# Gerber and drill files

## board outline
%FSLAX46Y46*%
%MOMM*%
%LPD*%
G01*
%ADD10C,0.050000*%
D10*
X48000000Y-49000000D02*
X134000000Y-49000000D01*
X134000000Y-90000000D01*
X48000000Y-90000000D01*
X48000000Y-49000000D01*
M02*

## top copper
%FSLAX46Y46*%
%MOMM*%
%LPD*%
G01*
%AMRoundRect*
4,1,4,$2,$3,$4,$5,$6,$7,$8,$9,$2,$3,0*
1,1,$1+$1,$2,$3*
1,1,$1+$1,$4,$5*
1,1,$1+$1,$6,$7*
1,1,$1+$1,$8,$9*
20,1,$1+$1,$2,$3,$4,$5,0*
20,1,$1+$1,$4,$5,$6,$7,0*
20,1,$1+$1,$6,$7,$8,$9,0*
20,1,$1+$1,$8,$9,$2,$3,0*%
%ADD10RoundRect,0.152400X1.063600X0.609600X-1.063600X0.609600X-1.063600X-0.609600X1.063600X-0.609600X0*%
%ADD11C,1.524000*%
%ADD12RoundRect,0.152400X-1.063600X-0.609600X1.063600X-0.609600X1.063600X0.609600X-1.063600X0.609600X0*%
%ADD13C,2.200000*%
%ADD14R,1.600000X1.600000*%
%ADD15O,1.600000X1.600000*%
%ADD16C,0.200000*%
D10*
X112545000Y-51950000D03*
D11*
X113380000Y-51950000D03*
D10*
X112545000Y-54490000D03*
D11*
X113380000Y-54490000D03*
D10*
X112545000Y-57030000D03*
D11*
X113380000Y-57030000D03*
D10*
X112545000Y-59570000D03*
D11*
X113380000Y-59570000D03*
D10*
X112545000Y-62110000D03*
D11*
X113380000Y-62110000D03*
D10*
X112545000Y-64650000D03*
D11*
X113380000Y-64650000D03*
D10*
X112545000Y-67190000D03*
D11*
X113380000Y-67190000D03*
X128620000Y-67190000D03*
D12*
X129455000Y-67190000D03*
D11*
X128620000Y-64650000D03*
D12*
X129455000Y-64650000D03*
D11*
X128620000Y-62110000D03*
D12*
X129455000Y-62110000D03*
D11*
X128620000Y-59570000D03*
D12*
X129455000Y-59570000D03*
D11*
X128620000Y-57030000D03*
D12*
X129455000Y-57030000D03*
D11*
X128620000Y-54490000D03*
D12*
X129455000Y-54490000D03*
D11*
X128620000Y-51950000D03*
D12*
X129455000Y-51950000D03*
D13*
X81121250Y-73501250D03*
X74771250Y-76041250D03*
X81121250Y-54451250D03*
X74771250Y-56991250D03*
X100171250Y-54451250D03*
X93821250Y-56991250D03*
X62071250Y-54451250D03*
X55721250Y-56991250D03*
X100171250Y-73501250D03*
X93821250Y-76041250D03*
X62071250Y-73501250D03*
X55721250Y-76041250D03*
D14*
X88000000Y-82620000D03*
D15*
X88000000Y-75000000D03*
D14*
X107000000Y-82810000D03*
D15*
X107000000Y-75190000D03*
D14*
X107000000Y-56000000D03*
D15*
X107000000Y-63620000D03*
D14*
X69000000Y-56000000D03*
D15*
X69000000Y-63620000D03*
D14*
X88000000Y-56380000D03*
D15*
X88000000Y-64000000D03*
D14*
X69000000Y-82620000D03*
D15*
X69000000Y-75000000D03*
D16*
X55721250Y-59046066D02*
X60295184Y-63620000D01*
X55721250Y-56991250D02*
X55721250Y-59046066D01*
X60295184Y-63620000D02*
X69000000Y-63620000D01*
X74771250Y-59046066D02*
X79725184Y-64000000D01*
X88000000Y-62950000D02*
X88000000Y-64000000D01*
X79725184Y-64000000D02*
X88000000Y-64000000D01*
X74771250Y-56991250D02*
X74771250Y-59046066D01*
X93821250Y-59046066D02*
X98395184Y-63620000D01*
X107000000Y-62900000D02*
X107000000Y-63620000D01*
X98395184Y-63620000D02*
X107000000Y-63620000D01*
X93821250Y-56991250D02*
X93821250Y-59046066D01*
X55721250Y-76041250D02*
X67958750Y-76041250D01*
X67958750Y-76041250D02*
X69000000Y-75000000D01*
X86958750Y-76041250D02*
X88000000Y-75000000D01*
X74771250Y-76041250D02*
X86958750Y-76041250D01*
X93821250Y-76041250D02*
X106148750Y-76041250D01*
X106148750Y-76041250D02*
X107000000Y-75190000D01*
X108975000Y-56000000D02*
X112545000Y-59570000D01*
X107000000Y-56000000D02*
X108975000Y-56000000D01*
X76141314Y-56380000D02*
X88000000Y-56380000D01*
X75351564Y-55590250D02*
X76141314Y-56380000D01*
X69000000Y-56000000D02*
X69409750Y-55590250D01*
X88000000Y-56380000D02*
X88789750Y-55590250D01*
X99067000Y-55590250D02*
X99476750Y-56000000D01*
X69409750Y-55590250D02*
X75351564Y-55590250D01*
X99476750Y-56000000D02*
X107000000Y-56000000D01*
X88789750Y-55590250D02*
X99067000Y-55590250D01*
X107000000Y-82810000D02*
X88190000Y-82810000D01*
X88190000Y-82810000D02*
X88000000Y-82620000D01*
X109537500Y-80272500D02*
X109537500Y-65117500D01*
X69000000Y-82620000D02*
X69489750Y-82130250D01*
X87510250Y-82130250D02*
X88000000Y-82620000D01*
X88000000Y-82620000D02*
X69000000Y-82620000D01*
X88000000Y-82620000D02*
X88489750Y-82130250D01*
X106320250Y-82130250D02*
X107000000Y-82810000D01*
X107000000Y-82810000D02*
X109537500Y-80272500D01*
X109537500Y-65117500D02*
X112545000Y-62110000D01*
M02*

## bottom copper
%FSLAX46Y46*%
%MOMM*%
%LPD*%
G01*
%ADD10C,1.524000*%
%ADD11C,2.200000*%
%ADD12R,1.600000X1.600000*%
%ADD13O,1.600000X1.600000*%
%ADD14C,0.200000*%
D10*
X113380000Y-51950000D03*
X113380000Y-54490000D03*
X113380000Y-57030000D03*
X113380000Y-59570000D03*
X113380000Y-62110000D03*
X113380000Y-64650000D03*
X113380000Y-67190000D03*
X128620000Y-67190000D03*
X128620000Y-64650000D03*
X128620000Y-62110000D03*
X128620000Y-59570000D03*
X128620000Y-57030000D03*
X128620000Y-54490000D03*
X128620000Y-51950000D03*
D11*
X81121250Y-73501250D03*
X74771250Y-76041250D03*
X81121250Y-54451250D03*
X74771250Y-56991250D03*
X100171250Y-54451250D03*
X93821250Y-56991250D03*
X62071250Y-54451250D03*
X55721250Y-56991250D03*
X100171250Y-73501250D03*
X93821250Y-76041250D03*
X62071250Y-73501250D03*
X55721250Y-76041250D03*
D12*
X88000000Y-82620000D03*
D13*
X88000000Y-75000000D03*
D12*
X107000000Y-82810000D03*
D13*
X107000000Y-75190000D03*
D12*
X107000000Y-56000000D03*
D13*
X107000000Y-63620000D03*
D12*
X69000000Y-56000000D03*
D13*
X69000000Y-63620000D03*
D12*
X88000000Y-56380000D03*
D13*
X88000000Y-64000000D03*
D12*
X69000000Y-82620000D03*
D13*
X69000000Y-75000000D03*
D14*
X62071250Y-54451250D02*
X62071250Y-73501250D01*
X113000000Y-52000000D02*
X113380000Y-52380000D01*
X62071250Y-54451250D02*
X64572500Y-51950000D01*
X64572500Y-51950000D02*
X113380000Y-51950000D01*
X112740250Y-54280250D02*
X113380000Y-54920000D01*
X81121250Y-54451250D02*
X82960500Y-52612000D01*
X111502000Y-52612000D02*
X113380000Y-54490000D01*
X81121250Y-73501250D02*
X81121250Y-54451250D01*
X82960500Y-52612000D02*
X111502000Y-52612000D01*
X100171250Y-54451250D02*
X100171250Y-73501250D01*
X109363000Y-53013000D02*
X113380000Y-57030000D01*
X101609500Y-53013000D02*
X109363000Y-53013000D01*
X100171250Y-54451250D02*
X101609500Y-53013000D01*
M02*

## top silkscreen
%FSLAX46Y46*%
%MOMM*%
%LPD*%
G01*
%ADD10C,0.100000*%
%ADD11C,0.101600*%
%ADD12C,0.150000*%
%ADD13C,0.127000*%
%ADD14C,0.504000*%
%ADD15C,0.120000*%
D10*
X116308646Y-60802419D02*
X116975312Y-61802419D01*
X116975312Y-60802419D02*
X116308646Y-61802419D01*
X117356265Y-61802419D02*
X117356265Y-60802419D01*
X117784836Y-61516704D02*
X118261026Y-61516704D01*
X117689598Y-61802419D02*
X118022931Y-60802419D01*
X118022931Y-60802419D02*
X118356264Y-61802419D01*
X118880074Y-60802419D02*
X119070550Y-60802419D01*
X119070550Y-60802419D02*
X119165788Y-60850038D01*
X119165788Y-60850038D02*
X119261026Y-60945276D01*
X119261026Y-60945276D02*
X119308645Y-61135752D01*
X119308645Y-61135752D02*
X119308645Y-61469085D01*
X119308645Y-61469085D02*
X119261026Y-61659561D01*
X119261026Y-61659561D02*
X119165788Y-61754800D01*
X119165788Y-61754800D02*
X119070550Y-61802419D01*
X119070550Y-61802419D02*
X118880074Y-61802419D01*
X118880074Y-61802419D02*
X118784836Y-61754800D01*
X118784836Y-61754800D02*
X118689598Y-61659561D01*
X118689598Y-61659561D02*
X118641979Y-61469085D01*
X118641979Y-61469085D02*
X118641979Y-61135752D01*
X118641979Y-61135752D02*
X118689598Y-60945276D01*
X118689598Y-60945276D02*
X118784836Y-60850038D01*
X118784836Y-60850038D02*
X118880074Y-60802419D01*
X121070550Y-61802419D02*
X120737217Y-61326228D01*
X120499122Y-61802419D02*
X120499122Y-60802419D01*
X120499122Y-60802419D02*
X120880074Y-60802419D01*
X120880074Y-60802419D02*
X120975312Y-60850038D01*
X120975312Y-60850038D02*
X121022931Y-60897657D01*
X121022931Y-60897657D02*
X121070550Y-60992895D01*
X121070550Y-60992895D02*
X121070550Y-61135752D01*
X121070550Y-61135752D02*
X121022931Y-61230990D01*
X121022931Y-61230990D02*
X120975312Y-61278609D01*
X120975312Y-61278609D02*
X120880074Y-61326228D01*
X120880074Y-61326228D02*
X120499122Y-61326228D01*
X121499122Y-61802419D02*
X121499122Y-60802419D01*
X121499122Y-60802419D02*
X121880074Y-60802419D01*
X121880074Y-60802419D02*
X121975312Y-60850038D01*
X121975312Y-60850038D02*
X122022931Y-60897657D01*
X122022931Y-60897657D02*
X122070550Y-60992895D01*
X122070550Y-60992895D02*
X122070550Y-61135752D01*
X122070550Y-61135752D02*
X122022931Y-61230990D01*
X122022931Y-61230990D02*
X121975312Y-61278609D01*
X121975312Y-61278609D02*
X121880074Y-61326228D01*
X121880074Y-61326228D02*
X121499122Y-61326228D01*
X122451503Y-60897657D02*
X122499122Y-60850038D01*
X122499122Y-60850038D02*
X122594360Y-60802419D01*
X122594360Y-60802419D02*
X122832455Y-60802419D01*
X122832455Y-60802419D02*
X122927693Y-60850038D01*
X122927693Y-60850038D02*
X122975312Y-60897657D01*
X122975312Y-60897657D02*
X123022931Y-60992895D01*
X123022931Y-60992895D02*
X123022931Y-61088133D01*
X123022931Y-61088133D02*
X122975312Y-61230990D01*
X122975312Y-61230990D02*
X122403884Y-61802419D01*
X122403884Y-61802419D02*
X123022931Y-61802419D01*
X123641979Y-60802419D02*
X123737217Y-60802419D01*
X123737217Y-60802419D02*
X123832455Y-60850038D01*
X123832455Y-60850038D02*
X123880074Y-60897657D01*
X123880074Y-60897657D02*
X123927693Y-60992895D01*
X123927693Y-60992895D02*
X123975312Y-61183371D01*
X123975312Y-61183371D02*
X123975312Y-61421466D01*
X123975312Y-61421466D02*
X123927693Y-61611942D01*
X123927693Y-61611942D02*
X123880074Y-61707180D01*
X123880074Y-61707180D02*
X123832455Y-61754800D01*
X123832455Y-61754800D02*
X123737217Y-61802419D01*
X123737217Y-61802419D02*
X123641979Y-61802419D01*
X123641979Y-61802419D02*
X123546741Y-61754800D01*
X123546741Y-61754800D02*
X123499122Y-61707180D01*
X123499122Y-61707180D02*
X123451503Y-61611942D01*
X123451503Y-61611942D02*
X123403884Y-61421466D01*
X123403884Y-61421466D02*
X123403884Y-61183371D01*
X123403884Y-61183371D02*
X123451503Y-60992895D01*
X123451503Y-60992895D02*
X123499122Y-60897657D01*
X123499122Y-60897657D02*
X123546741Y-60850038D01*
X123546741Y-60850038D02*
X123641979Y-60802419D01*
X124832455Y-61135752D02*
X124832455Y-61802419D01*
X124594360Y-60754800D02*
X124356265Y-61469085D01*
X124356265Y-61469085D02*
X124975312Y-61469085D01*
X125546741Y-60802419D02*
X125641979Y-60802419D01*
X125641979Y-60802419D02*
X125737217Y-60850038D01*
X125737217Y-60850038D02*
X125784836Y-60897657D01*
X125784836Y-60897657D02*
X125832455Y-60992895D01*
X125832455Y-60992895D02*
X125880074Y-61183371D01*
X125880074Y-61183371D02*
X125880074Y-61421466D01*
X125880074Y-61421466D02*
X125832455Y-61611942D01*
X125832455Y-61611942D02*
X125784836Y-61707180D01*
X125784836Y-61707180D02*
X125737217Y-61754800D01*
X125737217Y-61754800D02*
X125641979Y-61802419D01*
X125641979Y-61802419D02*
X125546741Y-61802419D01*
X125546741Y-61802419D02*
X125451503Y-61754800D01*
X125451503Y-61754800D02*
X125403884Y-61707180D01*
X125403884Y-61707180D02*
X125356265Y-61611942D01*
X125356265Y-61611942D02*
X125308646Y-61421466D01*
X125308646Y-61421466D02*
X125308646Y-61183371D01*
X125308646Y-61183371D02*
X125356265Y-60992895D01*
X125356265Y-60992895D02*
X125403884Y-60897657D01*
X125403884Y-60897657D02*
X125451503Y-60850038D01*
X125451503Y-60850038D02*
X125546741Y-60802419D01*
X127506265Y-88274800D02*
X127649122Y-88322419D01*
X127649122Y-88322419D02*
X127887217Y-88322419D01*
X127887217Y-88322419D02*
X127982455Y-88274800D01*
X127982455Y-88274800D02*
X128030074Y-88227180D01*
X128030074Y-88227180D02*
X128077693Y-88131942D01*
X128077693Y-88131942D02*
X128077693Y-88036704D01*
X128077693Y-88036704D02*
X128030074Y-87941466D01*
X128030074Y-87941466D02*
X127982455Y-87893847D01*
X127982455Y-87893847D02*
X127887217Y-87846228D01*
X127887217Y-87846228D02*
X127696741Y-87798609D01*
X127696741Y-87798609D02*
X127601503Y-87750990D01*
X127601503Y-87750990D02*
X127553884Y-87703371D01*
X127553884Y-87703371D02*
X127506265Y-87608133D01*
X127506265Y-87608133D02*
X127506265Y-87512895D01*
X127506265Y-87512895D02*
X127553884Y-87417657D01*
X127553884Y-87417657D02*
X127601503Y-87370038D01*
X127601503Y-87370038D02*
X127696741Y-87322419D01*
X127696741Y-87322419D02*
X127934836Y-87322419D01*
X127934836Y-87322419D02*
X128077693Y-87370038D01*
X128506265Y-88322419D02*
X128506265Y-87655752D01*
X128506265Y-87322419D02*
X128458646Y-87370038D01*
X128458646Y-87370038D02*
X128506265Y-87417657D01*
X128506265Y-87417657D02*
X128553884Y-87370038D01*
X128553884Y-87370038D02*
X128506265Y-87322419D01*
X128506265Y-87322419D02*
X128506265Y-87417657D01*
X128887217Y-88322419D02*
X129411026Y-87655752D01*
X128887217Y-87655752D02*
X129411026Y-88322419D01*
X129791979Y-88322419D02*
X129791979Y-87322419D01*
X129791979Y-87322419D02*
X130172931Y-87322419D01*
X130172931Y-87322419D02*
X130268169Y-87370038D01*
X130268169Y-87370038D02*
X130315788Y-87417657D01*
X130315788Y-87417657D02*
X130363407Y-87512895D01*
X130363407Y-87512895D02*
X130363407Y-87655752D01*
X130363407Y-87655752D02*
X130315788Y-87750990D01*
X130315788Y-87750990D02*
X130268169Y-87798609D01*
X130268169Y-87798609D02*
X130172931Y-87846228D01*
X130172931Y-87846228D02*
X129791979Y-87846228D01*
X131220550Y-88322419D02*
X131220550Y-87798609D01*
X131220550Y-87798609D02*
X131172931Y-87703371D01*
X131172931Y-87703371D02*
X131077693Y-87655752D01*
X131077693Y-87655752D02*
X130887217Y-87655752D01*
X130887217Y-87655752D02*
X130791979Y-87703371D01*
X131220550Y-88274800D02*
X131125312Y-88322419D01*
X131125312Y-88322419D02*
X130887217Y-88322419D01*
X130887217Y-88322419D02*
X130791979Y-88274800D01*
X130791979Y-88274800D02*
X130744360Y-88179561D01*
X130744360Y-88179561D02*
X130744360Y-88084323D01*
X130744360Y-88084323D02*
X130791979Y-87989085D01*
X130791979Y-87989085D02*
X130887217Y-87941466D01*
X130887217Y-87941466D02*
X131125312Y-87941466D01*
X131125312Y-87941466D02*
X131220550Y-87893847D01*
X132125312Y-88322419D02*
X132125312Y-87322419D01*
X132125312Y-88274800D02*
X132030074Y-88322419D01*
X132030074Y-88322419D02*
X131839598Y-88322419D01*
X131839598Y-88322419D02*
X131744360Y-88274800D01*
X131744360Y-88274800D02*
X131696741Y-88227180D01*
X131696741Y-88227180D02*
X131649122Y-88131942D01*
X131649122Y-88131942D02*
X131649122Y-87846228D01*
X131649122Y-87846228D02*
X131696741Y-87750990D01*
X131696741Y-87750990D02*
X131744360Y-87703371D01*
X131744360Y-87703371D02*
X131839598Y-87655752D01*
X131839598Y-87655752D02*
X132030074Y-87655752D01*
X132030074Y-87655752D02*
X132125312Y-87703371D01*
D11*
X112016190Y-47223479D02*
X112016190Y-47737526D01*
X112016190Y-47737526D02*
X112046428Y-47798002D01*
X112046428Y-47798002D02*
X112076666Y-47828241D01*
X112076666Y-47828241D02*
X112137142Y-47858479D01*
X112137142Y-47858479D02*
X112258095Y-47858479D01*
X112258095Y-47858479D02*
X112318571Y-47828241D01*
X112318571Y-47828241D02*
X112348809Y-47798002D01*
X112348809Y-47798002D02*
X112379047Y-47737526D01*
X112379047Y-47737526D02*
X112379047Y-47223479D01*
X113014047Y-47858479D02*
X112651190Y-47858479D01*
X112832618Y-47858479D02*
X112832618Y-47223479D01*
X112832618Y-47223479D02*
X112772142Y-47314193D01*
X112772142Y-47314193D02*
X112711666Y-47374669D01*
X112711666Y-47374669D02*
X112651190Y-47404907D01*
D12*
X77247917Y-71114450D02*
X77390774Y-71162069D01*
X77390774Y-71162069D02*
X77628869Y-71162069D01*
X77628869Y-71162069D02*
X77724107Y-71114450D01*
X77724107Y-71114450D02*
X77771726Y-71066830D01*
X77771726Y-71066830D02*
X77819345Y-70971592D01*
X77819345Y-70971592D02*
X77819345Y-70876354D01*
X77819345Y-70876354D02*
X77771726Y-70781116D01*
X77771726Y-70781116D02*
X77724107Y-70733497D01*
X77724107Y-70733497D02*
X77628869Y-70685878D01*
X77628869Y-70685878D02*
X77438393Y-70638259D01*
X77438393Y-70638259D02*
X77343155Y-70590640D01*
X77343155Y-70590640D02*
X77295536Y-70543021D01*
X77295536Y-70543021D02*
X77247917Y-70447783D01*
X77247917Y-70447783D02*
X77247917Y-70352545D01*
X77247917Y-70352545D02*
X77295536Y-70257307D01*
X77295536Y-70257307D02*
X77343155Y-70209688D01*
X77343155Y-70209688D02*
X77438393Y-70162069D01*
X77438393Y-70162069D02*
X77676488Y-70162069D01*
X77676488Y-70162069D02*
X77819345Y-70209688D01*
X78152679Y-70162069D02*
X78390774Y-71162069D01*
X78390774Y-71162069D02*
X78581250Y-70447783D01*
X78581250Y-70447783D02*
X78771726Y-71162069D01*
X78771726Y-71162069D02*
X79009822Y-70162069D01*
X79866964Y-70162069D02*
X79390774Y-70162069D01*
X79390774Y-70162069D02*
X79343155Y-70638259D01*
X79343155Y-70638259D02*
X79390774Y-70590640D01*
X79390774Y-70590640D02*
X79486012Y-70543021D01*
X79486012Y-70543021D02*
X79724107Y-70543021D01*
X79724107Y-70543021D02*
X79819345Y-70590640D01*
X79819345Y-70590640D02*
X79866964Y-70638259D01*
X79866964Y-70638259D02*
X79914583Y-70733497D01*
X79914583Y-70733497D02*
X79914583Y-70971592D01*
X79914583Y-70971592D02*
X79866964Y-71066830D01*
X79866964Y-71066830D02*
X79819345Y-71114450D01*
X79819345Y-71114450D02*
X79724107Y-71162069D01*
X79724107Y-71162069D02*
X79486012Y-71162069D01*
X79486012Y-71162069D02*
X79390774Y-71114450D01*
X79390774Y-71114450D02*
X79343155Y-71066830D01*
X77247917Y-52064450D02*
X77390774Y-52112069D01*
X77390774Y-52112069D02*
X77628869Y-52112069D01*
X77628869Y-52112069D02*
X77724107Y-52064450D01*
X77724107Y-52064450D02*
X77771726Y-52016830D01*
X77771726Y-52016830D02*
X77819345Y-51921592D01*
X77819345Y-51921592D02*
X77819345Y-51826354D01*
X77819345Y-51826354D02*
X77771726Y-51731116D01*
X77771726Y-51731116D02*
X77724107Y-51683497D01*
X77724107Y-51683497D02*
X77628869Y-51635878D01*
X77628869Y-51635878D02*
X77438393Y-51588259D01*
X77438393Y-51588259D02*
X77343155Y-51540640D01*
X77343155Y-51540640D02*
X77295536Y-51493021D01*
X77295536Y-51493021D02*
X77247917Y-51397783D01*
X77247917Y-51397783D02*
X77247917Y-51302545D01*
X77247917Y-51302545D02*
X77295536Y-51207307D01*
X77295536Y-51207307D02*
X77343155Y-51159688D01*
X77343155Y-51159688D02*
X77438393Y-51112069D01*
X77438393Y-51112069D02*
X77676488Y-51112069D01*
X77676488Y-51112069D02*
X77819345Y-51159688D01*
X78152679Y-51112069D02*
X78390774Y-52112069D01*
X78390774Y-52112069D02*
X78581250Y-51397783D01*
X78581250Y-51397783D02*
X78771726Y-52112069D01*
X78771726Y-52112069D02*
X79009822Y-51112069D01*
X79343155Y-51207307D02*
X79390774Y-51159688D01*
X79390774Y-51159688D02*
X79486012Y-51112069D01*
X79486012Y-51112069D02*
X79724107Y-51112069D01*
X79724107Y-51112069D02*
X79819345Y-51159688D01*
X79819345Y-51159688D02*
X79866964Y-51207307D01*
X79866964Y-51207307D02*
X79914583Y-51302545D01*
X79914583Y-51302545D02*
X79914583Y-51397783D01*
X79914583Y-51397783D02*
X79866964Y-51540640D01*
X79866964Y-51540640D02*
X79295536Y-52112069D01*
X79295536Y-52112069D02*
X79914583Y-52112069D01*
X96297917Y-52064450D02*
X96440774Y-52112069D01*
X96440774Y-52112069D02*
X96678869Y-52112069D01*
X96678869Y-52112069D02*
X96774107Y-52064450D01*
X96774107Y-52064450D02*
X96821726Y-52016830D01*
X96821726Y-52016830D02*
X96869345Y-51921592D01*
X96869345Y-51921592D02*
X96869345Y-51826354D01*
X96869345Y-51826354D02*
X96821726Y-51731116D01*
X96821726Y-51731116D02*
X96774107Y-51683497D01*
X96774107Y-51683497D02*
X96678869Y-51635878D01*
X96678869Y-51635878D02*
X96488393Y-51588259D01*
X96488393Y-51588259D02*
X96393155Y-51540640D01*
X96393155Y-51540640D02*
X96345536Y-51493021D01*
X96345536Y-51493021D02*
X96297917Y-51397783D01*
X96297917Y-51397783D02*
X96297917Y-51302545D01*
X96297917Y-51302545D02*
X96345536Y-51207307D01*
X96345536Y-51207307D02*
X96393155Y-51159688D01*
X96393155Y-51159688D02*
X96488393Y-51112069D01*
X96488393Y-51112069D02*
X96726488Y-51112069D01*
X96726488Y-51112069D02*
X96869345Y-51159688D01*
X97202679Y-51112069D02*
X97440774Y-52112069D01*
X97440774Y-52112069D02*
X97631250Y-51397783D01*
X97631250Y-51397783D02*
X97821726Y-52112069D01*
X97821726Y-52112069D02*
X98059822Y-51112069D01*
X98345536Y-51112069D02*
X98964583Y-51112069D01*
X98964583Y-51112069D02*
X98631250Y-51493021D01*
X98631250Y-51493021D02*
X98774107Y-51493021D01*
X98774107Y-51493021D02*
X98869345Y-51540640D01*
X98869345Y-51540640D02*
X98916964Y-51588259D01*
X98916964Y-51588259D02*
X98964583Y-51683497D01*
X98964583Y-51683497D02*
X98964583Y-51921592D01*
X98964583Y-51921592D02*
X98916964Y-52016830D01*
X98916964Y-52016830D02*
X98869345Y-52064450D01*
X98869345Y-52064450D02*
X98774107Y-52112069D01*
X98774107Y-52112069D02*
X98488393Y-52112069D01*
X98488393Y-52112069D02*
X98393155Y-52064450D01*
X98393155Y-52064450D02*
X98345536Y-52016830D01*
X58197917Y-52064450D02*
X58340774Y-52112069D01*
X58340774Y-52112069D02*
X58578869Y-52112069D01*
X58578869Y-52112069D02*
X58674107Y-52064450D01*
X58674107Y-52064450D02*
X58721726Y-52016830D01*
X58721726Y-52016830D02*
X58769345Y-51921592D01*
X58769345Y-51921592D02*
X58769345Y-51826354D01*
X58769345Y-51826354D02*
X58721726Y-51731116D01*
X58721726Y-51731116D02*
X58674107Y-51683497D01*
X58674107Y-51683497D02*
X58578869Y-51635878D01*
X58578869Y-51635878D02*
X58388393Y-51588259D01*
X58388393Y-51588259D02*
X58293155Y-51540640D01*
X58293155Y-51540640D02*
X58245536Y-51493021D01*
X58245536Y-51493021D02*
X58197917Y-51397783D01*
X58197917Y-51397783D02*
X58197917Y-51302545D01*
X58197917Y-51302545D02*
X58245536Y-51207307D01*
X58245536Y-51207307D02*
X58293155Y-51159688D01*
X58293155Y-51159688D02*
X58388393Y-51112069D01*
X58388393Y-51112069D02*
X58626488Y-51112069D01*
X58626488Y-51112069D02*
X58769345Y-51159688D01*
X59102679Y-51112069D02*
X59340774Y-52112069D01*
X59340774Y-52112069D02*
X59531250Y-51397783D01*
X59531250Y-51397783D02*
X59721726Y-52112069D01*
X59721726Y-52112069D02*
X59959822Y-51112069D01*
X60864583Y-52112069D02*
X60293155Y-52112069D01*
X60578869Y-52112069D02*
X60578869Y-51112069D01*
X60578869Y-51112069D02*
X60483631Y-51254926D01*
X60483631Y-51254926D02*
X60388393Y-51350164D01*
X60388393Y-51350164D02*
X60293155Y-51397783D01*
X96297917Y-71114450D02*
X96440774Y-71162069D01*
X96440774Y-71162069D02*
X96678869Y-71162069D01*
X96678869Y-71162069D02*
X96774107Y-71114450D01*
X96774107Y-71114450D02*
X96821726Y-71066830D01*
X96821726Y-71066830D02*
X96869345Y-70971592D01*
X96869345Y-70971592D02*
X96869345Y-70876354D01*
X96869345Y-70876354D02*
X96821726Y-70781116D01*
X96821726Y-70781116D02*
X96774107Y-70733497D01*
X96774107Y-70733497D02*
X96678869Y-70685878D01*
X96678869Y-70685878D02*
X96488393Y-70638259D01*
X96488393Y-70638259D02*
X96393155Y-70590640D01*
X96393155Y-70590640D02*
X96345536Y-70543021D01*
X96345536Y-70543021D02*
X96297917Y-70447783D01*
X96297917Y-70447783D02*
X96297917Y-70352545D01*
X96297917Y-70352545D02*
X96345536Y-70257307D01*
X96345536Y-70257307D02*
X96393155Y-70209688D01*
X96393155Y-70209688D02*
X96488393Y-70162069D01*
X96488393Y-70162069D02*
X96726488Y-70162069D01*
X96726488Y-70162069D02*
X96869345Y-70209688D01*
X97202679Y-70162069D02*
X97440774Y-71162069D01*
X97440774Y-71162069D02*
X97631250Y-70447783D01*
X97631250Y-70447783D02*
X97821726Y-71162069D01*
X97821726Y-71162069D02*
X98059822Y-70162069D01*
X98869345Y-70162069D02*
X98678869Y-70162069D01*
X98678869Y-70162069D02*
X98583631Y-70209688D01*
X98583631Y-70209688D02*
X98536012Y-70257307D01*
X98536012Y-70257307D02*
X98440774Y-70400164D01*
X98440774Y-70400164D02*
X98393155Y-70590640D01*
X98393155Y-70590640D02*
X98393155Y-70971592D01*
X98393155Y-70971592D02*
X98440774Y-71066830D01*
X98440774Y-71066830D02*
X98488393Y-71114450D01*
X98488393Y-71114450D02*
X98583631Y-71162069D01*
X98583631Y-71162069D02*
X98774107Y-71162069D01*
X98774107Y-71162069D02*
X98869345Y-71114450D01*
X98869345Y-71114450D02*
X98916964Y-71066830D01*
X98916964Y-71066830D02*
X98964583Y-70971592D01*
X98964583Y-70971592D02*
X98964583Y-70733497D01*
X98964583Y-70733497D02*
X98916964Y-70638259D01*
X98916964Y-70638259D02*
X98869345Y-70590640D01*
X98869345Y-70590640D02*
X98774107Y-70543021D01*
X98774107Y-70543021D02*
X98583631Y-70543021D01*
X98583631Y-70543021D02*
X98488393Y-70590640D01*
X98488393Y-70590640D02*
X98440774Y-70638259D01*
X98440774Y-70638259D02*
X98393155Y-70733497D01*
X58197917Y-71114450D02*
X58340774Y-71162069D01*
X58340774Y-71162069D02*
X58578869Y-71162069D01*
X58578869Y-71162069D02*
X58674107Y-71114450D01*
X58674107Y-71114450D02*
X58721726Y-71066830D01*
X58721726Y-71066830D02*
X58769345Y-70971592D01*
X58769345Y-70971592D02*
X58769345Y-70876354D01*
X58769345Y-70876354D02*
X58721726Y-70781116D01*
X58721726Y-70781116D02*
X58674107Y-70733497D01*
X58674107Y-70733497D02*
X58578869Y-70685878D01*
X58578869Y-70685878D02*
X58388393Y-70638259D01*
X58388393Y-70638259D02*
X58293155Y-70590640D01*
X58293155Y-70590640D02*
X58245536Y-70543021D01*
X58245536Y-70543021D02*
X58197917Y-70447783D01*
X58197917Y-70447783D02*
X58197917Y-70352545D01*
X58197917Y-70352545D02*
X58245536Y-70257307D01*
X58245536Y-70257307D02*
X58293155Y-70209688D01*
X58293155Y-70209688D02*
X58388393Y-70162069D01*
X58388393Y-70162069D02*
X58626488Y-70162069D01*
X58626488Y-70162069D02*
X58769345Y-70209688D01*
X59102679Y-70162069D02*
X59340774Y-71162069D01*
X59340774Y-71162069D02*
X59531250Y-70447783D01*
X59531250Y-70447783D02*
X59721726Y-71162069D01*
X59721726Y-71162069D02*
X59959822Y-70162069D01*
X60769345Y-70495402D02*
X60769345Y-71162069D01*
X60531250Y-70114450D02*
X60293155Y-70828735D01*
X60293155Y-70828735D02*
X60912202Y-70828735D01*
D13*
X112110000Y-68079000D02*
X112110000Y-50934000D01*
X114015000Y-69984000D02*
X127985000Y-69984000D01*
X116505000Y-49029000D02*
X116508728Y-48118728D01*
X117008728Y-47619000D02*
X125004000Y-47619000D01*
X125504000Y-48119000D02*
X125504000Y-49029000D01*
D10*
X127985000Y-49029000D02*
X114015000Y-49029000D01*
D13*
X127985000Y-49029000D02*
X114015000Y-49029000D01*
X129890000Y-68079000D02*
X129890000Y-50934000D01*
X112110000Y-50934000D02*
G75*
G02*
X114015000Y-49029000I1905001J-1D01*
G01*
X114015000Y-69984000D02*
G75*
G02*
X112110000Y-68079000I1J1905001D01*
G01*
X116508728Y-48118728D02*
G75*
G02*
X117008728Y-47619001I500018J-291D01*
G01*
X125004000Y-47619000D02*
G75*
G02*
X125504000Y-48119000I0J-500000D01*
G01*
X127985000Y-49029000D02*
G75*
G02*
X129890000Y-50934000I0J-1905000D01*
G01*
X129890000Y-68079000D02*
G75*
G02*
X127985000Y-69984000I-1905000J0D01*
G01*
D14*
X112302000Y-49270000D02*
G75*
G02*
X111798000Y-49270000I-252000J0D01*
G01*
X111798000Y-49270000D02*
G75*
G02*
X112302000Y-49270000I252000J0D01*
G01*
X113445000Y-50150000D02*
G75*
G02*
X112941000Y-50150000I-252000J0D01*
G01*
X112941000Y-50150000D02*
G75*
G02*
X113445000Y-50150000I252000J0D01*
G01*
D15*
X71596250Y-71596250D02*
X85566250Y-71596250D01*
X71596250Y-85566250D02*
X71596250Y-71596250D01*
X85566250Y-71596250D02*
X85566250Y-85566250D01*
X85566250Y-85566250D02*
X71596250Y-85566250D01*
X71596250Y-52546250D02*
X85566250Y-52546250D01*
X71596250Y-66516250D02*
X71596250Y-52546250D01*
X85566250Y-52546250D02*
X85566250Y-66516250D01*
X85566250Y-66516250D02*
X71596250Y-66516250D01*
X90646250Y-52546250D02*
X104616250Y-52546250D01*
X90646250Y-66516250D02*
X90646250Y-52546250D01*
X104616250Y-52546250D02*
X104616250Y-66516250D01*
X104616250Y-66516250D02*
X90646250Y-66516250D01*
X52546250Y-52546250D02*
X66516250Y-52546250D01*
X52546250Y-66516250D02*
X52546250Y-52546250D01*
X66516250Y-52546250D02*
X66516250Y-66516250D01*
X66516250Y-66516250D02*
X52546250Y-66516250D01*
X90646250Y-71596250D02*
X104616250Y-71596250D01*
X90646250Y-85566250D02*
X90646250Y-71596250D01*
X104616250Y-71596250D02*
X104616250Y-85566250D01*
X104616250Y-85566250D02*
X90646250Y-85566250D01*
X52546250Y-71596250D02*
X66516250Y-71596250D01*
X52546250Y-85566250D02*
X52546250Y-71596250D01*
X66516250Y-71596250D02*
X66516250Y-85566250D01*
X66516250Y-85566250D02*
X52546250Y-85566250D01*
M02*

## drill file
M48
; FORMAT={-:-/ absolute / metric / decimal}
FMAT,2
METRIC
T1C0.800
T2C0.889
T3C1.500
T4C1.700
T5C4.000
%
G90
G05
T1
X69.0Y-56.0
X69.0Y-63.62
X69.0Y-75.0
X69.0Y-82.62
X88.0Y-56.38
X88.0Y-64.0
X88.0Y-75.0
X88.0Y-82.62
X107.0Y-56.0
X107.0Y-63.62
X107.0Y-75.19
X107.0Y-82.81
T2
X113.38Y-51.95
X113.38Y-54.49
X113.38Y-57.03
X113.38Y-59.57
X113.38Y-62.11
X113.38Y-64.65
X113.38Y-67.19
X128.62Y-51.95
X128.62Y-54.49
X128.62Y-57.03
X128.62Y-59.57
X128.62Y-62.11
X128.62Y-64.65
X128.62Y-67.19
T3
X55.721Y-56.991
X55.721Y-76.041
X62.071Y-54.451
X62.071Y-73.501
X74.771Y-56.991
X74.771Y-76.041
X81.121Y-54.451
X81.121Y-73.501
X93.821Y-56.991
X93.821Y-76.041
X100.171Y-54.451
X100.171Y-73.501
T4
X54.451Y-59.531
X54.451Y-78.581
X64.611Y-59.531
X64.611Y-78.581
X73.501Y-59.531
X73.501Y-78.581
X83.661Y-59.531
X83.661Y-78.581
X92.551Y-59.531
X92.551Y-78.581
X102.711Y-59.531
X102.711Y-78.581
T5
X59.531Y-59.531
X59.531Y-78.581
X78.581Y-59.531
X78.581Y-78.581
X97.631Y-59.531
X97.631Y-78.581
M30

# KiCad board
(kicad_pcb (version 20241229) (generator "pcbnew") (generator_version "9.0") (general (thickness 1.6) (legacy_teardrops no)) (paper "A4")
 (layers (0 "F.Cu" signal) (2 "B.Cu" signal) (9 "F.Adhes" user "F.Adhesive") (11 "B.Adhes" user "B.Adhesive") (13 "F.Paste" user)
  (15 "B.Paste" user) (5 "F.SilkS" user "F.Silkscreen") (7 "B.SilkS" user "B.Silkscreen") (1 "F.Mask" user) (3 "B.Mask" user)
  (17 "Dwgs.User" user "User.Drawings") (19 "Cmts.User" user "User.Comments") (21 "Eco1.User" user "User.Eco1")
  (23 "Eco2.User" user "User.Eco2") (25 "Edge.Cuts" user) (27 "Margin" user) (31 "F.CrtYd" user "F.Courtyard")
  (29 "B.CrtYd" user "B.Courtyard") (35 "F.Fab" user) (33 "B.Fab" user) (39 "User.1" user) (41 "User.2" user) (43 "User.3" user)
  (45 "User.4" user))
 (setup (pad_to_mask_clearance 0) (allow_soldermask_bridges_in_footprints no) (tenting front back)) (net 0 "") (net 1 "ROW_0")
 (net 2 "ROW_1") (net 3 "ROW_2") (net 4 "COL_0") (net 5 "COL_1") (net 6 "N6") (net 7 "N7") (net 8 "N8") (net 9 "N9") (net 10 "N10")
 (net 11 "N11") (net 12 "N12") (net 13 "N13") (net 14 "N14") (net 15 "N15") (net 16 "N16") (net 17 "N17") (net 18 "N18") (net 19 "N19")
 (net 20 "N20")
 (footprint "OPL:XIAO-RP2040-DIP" (layer "F.Cu") (at 121 59.57)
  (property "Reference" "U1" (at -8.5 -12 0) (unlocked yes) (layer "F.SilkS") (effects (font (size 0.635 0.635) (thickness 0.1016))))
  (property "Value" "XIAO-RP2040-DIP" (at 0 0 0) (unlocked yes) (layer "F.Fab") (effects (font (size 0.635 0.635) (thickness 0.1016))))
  (fp_line (start -8.89 8.509) (end -8.89 -8.636) (stroke (width 0.127) (type solid)) (layer "F.SilkS"))
  (fp_line (start -6.985 10.414) (end 6.985 10.414) (stroke (width 0.127) (type solid)) (layer "F.SilkS"))
  (fp_line (start -4.495 -10.541) (end -4.491272 -11.451272) (stroke (width 0.127) (type solid)) (layer "F.SilkS"))
  (fp_line (start -3.991272 -11.951) (end 4.004 -11.951) (stroke (width 0.127) (type solid)) (layer "F.SilkS"))
  (fp_line (start 4.504 -11.451) (end 4.504 -10.541) (stroke (width 0.127) (type solid)) (layer "F.SilkS"))
  (fp_line (start 6.985 -10.541) (end -6.985 -10.541) (stroke (width 0.1) (type solid)) (layer "F.SilkS"))
  (fp_line (start 6.985 -10.541) (end -6.985 -10.541) (stroke (width 0.127) (type solid)) (layer "F.SilkS"))
  (fp_line (start 8.89 8.509) (end 8.89 -8.636) (stroke (width 0.127) (type solid)) (layer "F.SilkS"))
  (fp_arc (start -8.89 -8.636) (mid -8.332038 -9.983038) (end -6.985 -10.541) (stroke (width 0.127) (type solid)) (layer "F.SilkS"))
  (fp_arc (start -6.985 10.414) (mid -8.332038 9.856038) (end -8.89 8.509) (stroke (width 0.127) (type solid)) (layer "F.SilkS"))
  (fp_arc (start -4.491272 -11.451272) (mid -4.344728 -11.80464) (end -3.991272 -11.951) (stroke (width 0.127) (type default))
   (layer "F.SilkS"))
  (fp_arc (start 4.004 -11.951) (mid 4.357553 -11.804553) (end 4.504 -11.451) (stroke (width 0.127) (type default)) (layer "F.SilkS"))
  (fp_arc (start 6.985 -10.541) (mid 8.332038 -9.983038) (end 8.89 -8.636) (stroke (width 0.127) (type solid)) (layer "F.SilkS"))
  (fp_arc (start 8.89 8.509) (mid 8.332038 9.856038) (end 6.985 10.414) (stroke (width 0.127) (type solid)) (layer "F.SilkS"))
  (fp_circle (center -8.95 -10.3) (end -8.95 -10.554) (stroke (width 0.5) (type solid)) (fill yes) (layer "F.SilkS"))
  (fp_circle (center -7.807 -9.42) (end -7.807 -9.674) (stroke (width 0.5) (type solid)) (fill yes) (layer "F.SilkS"))
  (pad "1" smd roundrect (at -8.455 -7.62 180) (size 2.432 1.524) (layers "F.Cu" "F.Mask") (roundrect_rratio 0.1) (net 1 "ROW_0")
   (thermal_bridge_angle 45))
  (pad "1" thru_hole circle (at -7.62 -7.62 180) (size 1.524 1.524) (drill 0.889) (layers "*.Cu" "*.Mask") (remove_unused_layers no)
   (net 1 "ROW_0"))
  (pad "2" smd roundrect (at -8.455 -5.08 180) (size 2.432 1.524) (layers "F.Cu" "F.Mask") (roundrect_rratio 0.1) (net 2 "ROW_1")
   (thermal_bridge_angle 45))
  (pad "2" thru_hole circle (at -7.62 -5.08 180) (size 1.524 1.524) (drill 0.889) (layers "*.Cu" "*.Mask") (remove_unused_layers no)
   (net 2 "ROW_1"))
  (pad "3" smd roundrect (at -8.455 -2.54 180) (size 2.432 1.524) (layers "F.Cu" "F.Mask") (roundrect_rratio 0.1) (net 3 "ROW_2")
   (thermal_bridge_angle 45))
  (pad "3" thru_hole circle (at -7.62 -2.54 180) (size 1.524 1.524) (drill 0.889) (layers "*.Cu" "*.Mask") (remove_unused_layers no)
   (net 3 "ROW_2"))
  (pad "4" smd roundrect (at -8.455 0 180) (size 2.432 1.524) (layers "F.Cu" "F.Mask") (roundrect_rratio 0.1) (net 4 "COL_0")
   (thermal_bridge_angle 45))
  (pad "4" thru_hole circle (at -7.62 0 180) (size 1.524 1.524) (drill 0.889) (layers "*.Cu" "*.Mask") (remove_unused_layers no)
   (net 4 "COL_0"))
  (pad "5" smd roundrect (at -8.455 2.54 180) (size 2.432 1.524) (layers "F.Cu" "F.Mask") (roundrect_rratio 0.1) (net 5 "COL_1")
   (thermal_bridge_angle 45))
  (pad "5" thru_hole circle (at -7.62 2.54 180) (size 1.524 1.524) (drill 0.889) (layers "*.Cu" "*.Mask") (remove_unused_layers no)
   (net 5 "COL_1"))
  (pad "6" smd roundrect (at -8.455 5.08 180) (size 2.432 1.524) (layers "F.Cu" "F.Mask") (roundrect_rratio 0.1) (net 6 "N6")
   (thermal_bridge_angle 45))
  (pad "6" thru_hole circle (at -7.62 5.08 180) (size 1.524 1.524) (drill 0.889) (layers "*.Cu" "*.Mask") (remove_unused_layers no)
   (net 6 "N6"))
  (pad "7" smd roundrect (at -8.455 7.62 180) (size 2.432 1.524) (layers "F.Cu" "F.Mask") (roundrect_rratio 0.1) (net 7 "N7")
   (thermal_bridge_angle 45))
  (pad "7" thru_hole circle (at -7.62 7.62 180) (size 1.524 1.524) (drill 0.889) (layers "*.Cu" "*.Mask") (remove_unused_layers no)
   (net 7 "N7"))
  (pad "8" thru_hole circle (at 7.62 7.62) (size 1.524 1.524) (drill 0.889) (layers "*.Cu" "*.Mask") (remove_unused_layers no) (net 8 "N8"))
  (pad "8" smd roundrect (at 8.455 7.62) (size 2.432 1.524) (layers "F.Cu" "F.Mask") (roundrect_rratio 0.1) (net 8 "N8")
   (thermal_bridge_angle 45))
  (pad "9" thru_hole circle (at 7.62 5.08) (size 1.524 1.524) (drill 0.889) (layers "*.Cu" "*.Mask") (remove_unused_layers no) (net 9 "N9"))
  (pad "9" smd roundrect (at 8.455 5.08) (size 2.432 1.524) (layers "F.Cu" "F.Mask") (roundrect_rratio 0.1) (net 9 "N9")
   (thermal_bridge_angle 45))
  (pad "10" thru_hole circle (at 7.62 2.54) (size 1.524 1.524) (drill 0.889) (layers "*.Cu" "*.Mask") (remove_unused_layers no)
   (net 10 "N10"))
  (pad "10" smd roundrect (at 8.455 2.54) (size 2.432 1.524) (layers "F.Cu" "F.Mask") (roundrect_rratio 0.1) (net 10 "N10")
   (thermal_bridge_angle 45))
  (pad "11" thru_hole circle (at 7.62 0) (size 1.524 1.524) (drill 0.889) (layers "*.Cu" "*.Mask") (remove_unused_layers no) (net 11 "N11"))
  (pad "11" smd roundrect (at 8.455 0) (size 2.432 1.524) (layers "F.Cu" "F.Mask") (roundrect_rratio 0.1) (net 11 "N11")
   (thermal_bridge_angle 45))
  (pad "12" thru_hole circle (at 7.62 -2.54) (size 1.524 1.524) (drill 0.889) (layers "*.Cu" "*.Mask") (remove_unused_layers no)
   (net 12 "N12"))
  (pad "12" smd roundrect (at 8.455 -2.54) (size 2.432 1.524) (layers "F.Cu" "F.Mask") (roundrect_rratio 0.1) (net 12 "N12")
   (thermal_bridge_angle 45))
  (pad "13" thru_hole circle (at 7.62 -5.08) (size 1.524 1.524) (drill 0.889) (layers "*.Cu" "*.Mask") (remove_unused_layers no)
   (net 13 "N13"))
  (pad "13" smd roundrect (at 8.455 -5.08) (size 2.432 1.524) (layers "F.Cu" "F.Mask") (roundrect_rratio 0.1) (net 13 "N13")
   (thermal_bridge_angle 45))
  (pad "14" thru_hole circle (at 7.62 -7.62) (size 1.524 1.524) (drill 0.889) (layers "*.Cu" "*.Mask") (remove_unused_layers no)
   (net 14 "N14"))
  (pad "14" smd roundrect (at 8.455 -7.62) (size 2.432 1.524) (layers "F.Cu" "F.Mask") (roundrect_rratio 0.1) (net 14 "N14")
   (thermal_bridge_angle 45)))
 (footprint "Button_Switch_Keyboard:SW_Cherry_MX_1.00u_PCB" (layer "F.Cu") (at 81.12125 73.50125)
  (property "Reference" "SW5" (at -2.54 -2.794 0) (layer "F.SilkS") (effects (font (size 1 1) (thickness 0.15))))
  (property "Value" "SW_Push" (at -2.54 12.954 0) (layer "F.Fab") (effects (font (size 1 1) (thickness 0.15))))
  (fp_line (start -9.525 -1.905) (end 4.445 -1.905) (stroke (width 0.12) (type solid)) (layer "F.SilkS"))
  (fp_line (start -9.525 12.065) (end -9.525 -1.905) (stroke (width 0.12) (type solid)) (layer "F.SilkS"))
  (fp_line (start 4.445 -1.905) (end 4.445 12.065) (stroke (width 0.12) (type solid)) (layer "F.SilkS"))
  (fp_line (start 4.445 12.065) (end -9.525 12.065) (stroke (width 0.12) (type solid)) (layer "F.SilkS"))
  (pad "" np_thru_hole circle (at -7.62 5.08) (size 1.7 1.7) (drill 1.7) (layers "*.Cu" "*.Mask"))
  (pad "" np_thru_hole circle (at -2.54 5.08) (size 4 4) (drill 4) (layers "*.Cu" "*.Mask"))
  (pad "" np_thru_hole circle (at 2.54 5.08) (size 1.7 1.7) (drill 1.7) (layers "*.Cu" "*.Mask"))
  (pad "1" thru_hole circle (at 0 0) (size 2.2 2.2) (drill 1.5) (layers "*.Cu" "*.Mask") (remove_unused_layers no) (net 2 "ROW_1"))
  (pad "2" thru_hole circle (at -6.35 2.54) (size 2.2 2.2) (drill 1.5) (layers "*.Cu" "*.Mask") (remove_unused_layers no) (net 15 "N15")))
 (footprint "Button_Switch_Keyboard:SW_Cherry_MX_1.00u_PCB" (layer "F.Cu") (at 81.12125 54.45125)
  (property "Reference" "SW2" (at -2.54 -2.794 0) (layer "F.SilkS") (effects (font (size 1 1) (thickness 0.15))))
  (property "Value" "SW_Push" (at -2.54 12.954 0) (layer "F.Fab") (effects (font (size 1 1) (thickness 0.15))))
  (fp_line (start -9.525 -1.905) (end 4.445 -1.905) (stroke (width 0.12) (type solid)) (layer "F.SilkS"))
  (fp_line (start -9.525 12.065) (end -9.525 -1.905) (stroke (width 0.12) (type solid)) (layer "F.SilkS"))
  (fp_line (start 4.445 -1.905) (end 4.445 12.065) (stroke (width 0.12) (type solid)) (layer "F.SilkS"))
  (fp_line (start 4.445 12.065) (end -9.525 12.065) (stroke (width 0.12) (type solid)) (layer "F.SilkS"))
  (pad "" np_thru_hole circle (at -7.62 5.08) (size 1.7 1.7) (drill 1.7) (layers "*.Cu" "*.Mask"))
  (pad "" np_thru_hole circle (at -2.54 5.08) (size 4 4) (drill 4) (layers "*.Cu" "*.Mask"))
  (pad "" np_thru_hole circle (at 2.54 5.08) (size 1.7 1.7) (drill 1.7) (layers "*.Cu" "*.Mask"))
  (pad "1" thru_hole circle (at 0 0) (size 2.2 2.2) (drill 1.5) (layers "*.Cu" "*.Mask") (remove_unused_layers no) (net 2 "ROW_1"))
  (pad "2" thru_hole circle (at -6.35 2.54) (size 2.2 2.2) (drill 1.5) (layers "*.Cu" "*.Mask") (remove_unused_layers no) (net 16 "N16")))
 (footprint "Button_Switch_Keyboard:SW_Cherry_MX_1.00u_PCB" (layer "F.Cu") (at 100.17125 54.45125)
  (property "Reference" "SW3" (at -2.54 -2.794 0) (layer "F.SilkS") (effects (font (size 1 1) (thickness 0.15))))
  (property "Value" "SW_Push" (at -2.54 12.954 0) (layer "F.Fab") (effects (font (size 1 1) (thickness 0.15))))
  (fp_line (start -9.525 -1.905) (end 4.445 -1.905) (stroke (width 0.12) (type solid)) (layer "F.SilkS"))
  (fp_line (start -9.525 12.065) (end -9.525 -1.905) (stroke (width 0.12) (type solid)) (layer "F.SilkS"))
  (fp_line (start 4.445 -1.905) (end 4.445 12.065) (stroke (width 0.12) (type solid)) (layer "F.SilkS"))
  (fp_line (start 4.445 12.065) (end -9.525 12.065) (stroke (width 0.12) (type solid)) (layer "F.SilkS"))
  (pad "" np_thru_hole circle (at -7.62 5.08) (size 1.7 1.7) (drill 1.7) (layers "*.Cu" "*.Mask"))
  (pad "" np_thru_hole circle (at -2.54 5.08) (size 4 4) (drill 4) (layers "*.Cu" "*.Mask"))
  (pad "" np_thru_hole circle (at 2.54 5.08) (size 1.7 1.7) (drill 1.7) (layers "*.Cu" "*.Mask"))
  (pad "1" thru_hole circle (at 0 0) (size 2.2 2.2) (drill 1.5) (layers "*.Cu" "*.Mask") (remove_unused_layers no) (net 3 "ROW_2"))
  (pad "2" thru_hole circle (at -6.35 2.54) (size 2.2 2.2) (drill 1.5) (layers "*.Cu" "*.Mask") (remove_unused_layers no) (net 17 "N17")))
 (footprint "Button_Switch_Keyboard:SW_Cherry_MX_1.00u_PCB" (layer "F.Cu") (at 62.07125 54.45125)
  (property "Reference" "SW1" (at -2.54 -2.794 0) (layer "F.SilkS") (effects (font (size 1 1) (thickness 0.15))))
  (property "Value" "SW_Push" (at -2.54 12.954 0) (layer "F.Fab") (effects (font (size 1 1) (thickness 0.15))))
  (fp_line (start -9.525 -1.905) (end 4.445 -1.905) (stroke (width 0.12) (type solid)) (layer "F.SilkS"))
  (fp_line (start -9.525 12.065) (end -9.525 -1.905) (stroke (width 0.12) (type solid)) (layer "F.SilkS"))
  (fp_line (start 4.445 -1.905) (end 4.445 12.065) (stroke (width 0.12) (type solid)) (layer "F.SilkS"))
  (fp_line (start 4.445 12.065) (end -9.525 12.065) (stroke (width 0.12) (type solid)) (layer "F.SilkS"))
  (pad "" np_thru_hole circle (at -7.62 5.08) (size 1.7 1.7) (drill 1.7) (layers "*.Cu" "*.Mask"))
  (pad "" np_thru_hole circle (at -2.54 5.08) (size 4 4) (drill 4) (layers "*.Cu" "*.Mask"))
  (pad "" np_thru_hole circle (at 2.54 5.08) (size 1.7 1.7) (drill 1.7) (layers "*.Cu" "*.Mask"))
  (pad "1" thru_hole circle (at 0 0) (size 2.2 2.2) (drill 1.5) (layers "*.Cu" "*.Mask") (remove_unused_layers no) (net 1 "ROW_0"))
  (pad "2" thru_hole circle (at -6.35 2.54) (size 2.2 2.2) (drill 1.5) (layers "*.Cu" "*.Mask") (remove_unused_layers no) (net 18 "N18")))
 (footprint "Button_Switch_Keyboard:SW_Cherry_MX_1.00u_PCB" (layer "F.Cu") (at 100.17125 73.50125)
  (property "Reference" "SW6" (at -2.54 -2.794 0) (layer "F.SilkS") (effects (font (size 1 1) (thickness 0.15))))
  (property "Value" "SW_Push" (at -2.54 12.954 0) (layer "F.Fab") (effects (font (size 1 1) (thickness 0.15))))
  (fp_line (start -9.525 -1.905) (end 4.445 -1.905) (stroke (width 0.12) (type solid)) (layer "F.SilkS"))
  (fp_line (start -9.525 12.065) (end -9.525 -1.905) (stroke (width 0.12) (type solid)) (layer "F.SilkS"))
  (fp_line (start 4.445 -1.905) (end 4.445 12.065) (stroke (width 0.12) (type solid)) (layer "F.SilkS"))
  (fp_line (start 4.445 12.065) (end -9.525 12.065) (stroke (width 0.12) (type solid)) (layer "F.SilkS"))
  (pad "" np_thru_hole circle (at -7.62 5.08) (size 1.7 1.7) (drill 1.7) (layers "*.Cu" "*.Mask"))
  (pad "" np_thru_hole circle (at -2.54 5.08) (size 4 4) (drill 4) (layers "*.Cu" "*.Mask"))
  (pad "" np_thru_hole circle (at 2.54 5.08) (size 1.7 1.7) (drill 1.7) (layers "*.Cu" "*.Mask"))
  (pad "1" thru_hole circle (at 0 0) (size 2.2 2.2) (drill 1.5) (layers "*.Cu" "*.Mask") (remove_unused_layers no) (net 3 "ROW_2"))
  (pad "2" thru_hole circle (at -6.35 2.54) (size 2.2 2.2) (drill 1.5) (layers "*.Cu" "*.Mask") (remove_unused_layers no) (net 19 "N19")))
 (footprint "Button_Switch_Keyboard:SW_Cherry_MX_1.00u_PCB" (layer "F.Cu") (at 62.07125 73.50125)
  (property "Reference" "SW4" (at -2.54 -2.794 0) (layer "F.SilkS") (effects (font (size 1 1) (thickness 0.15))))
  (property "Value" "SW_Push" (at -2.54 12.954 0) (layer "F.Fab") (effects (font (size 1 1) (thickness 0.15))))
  (fp_line (start -9.525 -1.905) (end 4.445 -1.905) (stroke (width 0.12) (type solid)) (layer "F.SilkS"))
  (fp_line (start -9.525 12.065) (end -9.525 -1.905) (stroke (width 0.12) (type solid)) (layer "F.SilkS"))
  (fp_line (start 4.445 -1.905) (end 4.445 12.065) (stroke (width 0.12) (type solid)) (layer "F.SilkS"))
  (fp_line (start 4.445 12.065) (end -9.525 12.065) (stroke (width 0.12) (type solid)) (layer "F.SilkS"))
  (pad "" np_thru_hole circle (at -7.62 5.08) (size 1.7 1.7) (drill 1.7) (layers "*.Cu" "*.Mask"))
  (pad "" np_thru_hole circle (at -2.54 5.08) (size 4 4) (drill 4) (layers "*.Cu" "*.Mask"))
  (pad "" np_thru_hole circle (at 2.54 5.08) (size 1.7 1.7) (drill 1.7) (layers "*.Cu" "*.Mask"))
  (pad "1" thru_hole circle (at 0 0) (size 2.2 2.2) (drill 1.5) (layers "*.Cu" "*.Mask") (remove_unused_layers no) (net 1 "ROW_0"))
  (pad "2" thru_hole circle (at -6.35 2.54) (size 2.2 2.2) (drill 1.5) (layers "*.Cu" "*.Mask") (remove_unused_layers no) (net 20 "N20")))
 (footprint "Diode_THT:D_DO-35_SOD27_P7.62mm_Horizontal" (layer "B.Cu") (at 88 82.62 90)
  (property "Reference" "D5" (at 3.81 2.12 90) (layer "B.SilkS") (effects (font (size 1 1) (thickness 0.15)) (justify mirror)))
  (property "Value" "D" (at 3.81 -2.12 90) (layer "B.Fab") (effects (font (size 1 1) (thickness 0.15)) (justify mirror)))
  (pad "1" thru_hole rect (at 0 0 90) (size 1.6 1.6) (drill 0.8) (layers "*.Cu" "*.Mask") (remove_unused_layers no) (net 5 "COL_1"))
  (pad "2" thru_hole oval (at 7.62 0 90) (size 1.6 1.6) (drill 0.8) (layers "*.Cu" "*.Mask") (remove_unused_layers no) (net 15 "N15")))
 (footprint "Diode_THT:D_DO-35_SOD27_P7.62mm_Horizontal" (layer "B.Cu") (at 107 82.81 90)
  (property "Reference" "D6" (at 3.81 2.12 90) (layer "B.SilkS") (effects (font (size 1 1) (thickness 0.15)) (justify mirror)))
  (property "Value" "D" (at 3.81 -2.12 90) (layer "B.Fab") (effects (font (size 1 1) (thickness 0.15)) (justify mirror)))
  (pad "1" thru_hole rect (at 0 0 90) (size 1.6 1.6) (drill 0.8) (layers "*.Cu" "*.Mask") (remove_unused_layers no) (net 5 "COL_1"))
  (pad "2" thru_hole oval (at 7.62 0 90) (size 1.6 1.6) (drill 0.8) (layers "*.Cu" "*.Mask") (remove_unused_layers no) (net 19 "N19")))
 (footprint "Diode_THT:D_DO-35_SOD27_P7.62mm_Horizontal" (layer "B.Cu") (at 107 56 -90)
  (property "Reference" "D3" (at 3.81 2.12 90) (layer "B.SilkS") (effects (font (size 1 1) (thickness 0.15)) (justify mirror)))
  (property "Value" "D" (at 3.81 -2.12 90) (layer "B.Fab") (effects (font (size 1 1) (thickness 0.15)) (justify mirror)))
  (pad "1" thru_hole rect (at 0 0 270) (size 1.6 1.6) (drill 0.8) (layers "*.Cu" "*.Mask") (remove_unused_layers no) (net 4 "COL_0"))
  (pad "2" thru_hole oval (at 7.62 0 270) (size 1.6 1.6) (drill 0.8) (layers "*.Cu" "*.Mask") (remove_unused_layers no) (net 17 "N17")))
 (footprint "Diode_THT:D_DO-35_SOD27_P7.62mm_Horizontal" (layer "B.Cu") (at 69 56 -90)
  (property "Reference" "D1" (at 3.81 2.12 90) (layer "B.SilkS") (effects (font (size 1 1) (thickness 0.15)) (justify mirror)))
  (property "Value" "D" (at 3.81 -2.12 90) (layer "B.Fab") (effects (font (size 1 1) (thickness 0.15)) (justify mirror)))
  (pad "1" thru_hole rect (at 0 0 270) (size 1.6 1.6) (drill 0.8) (layers "*.Cu" "*.Mask") (remove_unused_layers no) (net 4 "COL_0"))
  (pad "2" thru_hole oval (at 7.62 0 270) (size 1.6 1.6) (drill 0.8) (layers "*.Cu" "*.Mask") (remove_unused_layers no) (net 18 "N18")))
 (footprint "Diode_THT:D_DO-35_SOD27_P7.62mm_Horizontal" (layer "B.Cu") (at 88 56.38 -90)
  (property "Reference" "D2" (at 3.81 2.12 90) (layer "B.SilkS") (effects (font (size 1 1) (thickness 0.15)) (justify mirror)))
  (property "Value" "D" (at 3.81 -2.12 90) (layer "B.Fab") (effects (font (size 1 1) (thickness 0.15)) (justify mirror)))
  (pad "1" thru_hole rect (at 0 0 270) (size 1.6 1.6) (drill 0.8) (layers "*.Cu" "*.Mask") (remove_unused_layers no) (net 4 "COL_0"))
  (pad "2" thru_hole oval (at 7.62 0 270) (size 1.6 1.6) (drill 0.8) (layers "*.Cu" "*.Mask") (remove_unused_layers no) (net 16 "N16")))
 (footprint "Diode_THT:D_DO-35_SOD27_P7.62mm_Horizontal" (layer "B.Cu") (at 69 82.62 90)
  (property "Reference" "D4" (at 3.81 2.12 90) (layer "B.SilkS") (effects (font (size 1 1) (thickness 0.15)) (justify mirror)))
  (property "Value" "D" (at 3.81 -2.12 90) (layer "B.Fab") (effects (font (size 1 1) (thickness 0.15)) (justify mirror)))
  (pad "1" thru_hole rect (at 0 0 90) (size 1.6 1.6) (drill 0.8) (layers "*.Cu" "*.Mask") (remove_unused_layers no) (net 5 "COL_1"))
  (pad "2" thru_hole oval (at 7.62 0 90) (size 1.6 1.6) (drill 0.8) (layers "*.Cu" "*.Mask") (remove_unused_layers no) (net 20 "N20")))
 (gr_rect (start 48 49) (end 134 90) (stroke (width 0.05) (type default)) (fill no) (layer "Edge.Cuts"))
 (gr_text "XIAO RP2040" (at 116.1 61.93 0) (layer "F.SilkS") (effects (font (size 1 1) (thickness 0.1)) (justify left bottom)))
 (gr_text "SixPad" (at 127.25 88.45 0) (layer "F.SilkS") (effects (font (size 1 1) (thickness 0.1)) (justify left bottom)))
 (segment (start 62.07125 54.45125) (end 62.07125 73.50125) (width 0.2) (layer "B.Cu") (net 1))
 (segment (start 113 52) (end 113.38 52.38) (width 0.2) (layer "B.Cu") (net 1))
 (segment (start 62.07125 54.45125) (end 64.5725 51.95) (width 0.2) (layer "B.Cu") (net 1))
 (segment (start 64.5725 51.95) (end 113.38 51.95) (width 0.2) (layer "B.Cu") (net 1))
 (segment (start 55.72125 59.046066) (end 60.295184 63.62) (width 0.2) (layer "F.Cu") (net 18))
 (segment (start 55.72125 56.99125) (end 55.72125 59.046066) (width 0.2) (layer "F.Cu") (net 18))
 (segment (start 60.295184 63.62) (end 69 63.62) (width 0.2) (layer "F.Cu") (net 18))
 (segment (start 74.77125 59.046066) (end 79.725184 64) (width 0.2) (layer "F.Cu") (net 16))
 (segment (start 88 62.95) (end 88 64) (width 0.2) (layer "F.Cu") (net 16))
 (segment (start 79.725184 64) (end 88 64) (width 0.2) (layer "F.Cu") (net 16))
 (segment (start 74.77125 56.99125) (end 74.77125 59.046066) (width 0.2) (layer "F.Cu") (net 16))
 (segment (start 112.74025 54.28025) (end 113.38 54.92) (width 0.2) (layer "B.Cu") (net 2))
 (segment (start 81.12125 54.45125) (end 82.9605 52.612) (width 0.2) (layer "B.Cu") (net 2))
 (segment (start 111.502 52.612) (end 113.38 54.49) (width 0.2) (layer "B.Cu") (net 2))
 (segment (start 81.12125 73.50125) (end 81.12125 54.45125) (width 0.2) (layer "B.Cu") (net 2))
 (segment (start 82.9605 52.612) (end 111.502 52.612) (width 0.2) (layer "B.Cu") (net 2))
 (segment (start 93.82125 59.046066) (end 98.395184 63.62) (width 0.2) (layer "F.Cu") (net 17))
 (segment (start 107 62.9) (end 107 63.62) (width 0.2) (layer "F.Cu") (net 17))
 (segment (start 98.395184 63.62) (end 107 63.62) (width 0.2) (layer "F.Cu") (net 17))
 (segment (start 93.82125 56.99125) (end 93.82125 59.046066) (width 0.2) (layer "F.Cu") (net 17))
 (segment (start 100.17125 54.45125) (end 100.17125 73.50125) (width 0.2) (layer "B.Cu") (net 3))
 (segment (start 109.363 53.013) (end 113.38 57.03) (width 0.2) (layer "B.Cu") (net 3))
 (segment (start 101.6095 53.013) (end 109.363 53.013) (width 0.2) (layer "B.Cu") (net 3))
 (segment (start 100.17125 54.45125) (end 101.6095 53.013) (width 0.2) (layer "B.Cu") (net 3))
 (segment (start 55.72125 76.04125) (end 67.95875 76.04125) (width 0.2) (layer "F.Cu") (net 20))
 (segment (start 67.95875 76.04125) (end 69 75) (width 0.2) (layer "F.Cu") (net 20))
 (segment (start 86.95875 76.04125) (end 88 75) (width 0.2) (layer "F.Cu") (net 15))
 (segment (start 74.77125 76.04125) (end 86.95875 76.04125) (width 0.2) (layer "F.Cu") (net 15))
 (segment (start 93.82125 76.04125) (end 106.14875 76.04125) (width 0.2) (layer "F.Cu") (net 19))
 (segment (start 106.14875 76.04125) (end 107 75.19) (width 0.2) (layer "F.Cu") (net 19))
 (segment (start 108.975 56) (end 112.545 59.57) (width 0.2) (layer "F.Cu") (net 4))
 (segment (start 107 56) (end 108.975 56) (width 0.2) (layer "F.Cu") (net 4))
 (segment (start 76.141314 56.38) (end 88 56.38) (width 0.2) (layer "F.Cu") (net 4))
 (segment (start 75.351564 55.59025) (end 76.141314 56.38) (width 0.2) (layer "F.Cu") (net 4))
 (segment (start 69 56) (end 69.40975 55.59025) (width 0.2) (layer "F.Cu") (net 4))
 (segment (start 88 56.38) (end 88.78975 55.59025) (width 0.2) (layer "F.Cu") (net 4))
 (segment (start 99.067 55.59025) (end 99.47675 56) (width 0.2) (layer "F.Cu") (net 4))
 (segment (start 69.40975 55.59025) (end 75.351564 55.59025) (width 0.2) (layer "F.Cu") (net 4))
 (segment (start 99.47675 56) (end 107 56) (width 0.2) (layer "F.Cu") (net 4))
 (segment (start 88.78975 55.59025) (end 99.067 55.59025) (width 0.2) (layer "F.Cu") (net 4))
 (segment (start 107 82.81) (end 88.19 82.81) (width 0.2) (layer "F.Cu") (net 5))
 (segment (start 88.19 82.81) (end 88 82.62) (width 0.2) (layer "F.Cu") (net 5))
 (segment (start 109.5375 80.2725) (end 109.5375 65.1175) (width 0.2) (layer "F.Cu") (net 5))
 (segment (start 69 82.62) (end 69.48975 82.13025) (width 0.2) (layer "F.Cu") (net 5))
 (segment (start 87.51025 82.13025) (end 88 82.62) (width 0.2) (layer "F.Cu") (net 5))
 (segment (start 88 82.62) (end 69 82.62) (width 0.2) (layer "F.Cu") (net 5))
 (segment (start 88 82.62) (end 88.48975 82.13025) (width 0.2) (layer "F.Cu") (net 5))
 (segment (start 106.32025 82.13025) (end 107 82.81) (width 0.2) (layer "F.Cu") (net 5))
 (segment (start 107 82.81) (end 109.5375 80.2725) (width 0.2) (layer "F.Cu") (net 5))
 (segment (start 109.5375 65.1175) (end 112.545 62.11) (width 0.2) (layer "F.Cu") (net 5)))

